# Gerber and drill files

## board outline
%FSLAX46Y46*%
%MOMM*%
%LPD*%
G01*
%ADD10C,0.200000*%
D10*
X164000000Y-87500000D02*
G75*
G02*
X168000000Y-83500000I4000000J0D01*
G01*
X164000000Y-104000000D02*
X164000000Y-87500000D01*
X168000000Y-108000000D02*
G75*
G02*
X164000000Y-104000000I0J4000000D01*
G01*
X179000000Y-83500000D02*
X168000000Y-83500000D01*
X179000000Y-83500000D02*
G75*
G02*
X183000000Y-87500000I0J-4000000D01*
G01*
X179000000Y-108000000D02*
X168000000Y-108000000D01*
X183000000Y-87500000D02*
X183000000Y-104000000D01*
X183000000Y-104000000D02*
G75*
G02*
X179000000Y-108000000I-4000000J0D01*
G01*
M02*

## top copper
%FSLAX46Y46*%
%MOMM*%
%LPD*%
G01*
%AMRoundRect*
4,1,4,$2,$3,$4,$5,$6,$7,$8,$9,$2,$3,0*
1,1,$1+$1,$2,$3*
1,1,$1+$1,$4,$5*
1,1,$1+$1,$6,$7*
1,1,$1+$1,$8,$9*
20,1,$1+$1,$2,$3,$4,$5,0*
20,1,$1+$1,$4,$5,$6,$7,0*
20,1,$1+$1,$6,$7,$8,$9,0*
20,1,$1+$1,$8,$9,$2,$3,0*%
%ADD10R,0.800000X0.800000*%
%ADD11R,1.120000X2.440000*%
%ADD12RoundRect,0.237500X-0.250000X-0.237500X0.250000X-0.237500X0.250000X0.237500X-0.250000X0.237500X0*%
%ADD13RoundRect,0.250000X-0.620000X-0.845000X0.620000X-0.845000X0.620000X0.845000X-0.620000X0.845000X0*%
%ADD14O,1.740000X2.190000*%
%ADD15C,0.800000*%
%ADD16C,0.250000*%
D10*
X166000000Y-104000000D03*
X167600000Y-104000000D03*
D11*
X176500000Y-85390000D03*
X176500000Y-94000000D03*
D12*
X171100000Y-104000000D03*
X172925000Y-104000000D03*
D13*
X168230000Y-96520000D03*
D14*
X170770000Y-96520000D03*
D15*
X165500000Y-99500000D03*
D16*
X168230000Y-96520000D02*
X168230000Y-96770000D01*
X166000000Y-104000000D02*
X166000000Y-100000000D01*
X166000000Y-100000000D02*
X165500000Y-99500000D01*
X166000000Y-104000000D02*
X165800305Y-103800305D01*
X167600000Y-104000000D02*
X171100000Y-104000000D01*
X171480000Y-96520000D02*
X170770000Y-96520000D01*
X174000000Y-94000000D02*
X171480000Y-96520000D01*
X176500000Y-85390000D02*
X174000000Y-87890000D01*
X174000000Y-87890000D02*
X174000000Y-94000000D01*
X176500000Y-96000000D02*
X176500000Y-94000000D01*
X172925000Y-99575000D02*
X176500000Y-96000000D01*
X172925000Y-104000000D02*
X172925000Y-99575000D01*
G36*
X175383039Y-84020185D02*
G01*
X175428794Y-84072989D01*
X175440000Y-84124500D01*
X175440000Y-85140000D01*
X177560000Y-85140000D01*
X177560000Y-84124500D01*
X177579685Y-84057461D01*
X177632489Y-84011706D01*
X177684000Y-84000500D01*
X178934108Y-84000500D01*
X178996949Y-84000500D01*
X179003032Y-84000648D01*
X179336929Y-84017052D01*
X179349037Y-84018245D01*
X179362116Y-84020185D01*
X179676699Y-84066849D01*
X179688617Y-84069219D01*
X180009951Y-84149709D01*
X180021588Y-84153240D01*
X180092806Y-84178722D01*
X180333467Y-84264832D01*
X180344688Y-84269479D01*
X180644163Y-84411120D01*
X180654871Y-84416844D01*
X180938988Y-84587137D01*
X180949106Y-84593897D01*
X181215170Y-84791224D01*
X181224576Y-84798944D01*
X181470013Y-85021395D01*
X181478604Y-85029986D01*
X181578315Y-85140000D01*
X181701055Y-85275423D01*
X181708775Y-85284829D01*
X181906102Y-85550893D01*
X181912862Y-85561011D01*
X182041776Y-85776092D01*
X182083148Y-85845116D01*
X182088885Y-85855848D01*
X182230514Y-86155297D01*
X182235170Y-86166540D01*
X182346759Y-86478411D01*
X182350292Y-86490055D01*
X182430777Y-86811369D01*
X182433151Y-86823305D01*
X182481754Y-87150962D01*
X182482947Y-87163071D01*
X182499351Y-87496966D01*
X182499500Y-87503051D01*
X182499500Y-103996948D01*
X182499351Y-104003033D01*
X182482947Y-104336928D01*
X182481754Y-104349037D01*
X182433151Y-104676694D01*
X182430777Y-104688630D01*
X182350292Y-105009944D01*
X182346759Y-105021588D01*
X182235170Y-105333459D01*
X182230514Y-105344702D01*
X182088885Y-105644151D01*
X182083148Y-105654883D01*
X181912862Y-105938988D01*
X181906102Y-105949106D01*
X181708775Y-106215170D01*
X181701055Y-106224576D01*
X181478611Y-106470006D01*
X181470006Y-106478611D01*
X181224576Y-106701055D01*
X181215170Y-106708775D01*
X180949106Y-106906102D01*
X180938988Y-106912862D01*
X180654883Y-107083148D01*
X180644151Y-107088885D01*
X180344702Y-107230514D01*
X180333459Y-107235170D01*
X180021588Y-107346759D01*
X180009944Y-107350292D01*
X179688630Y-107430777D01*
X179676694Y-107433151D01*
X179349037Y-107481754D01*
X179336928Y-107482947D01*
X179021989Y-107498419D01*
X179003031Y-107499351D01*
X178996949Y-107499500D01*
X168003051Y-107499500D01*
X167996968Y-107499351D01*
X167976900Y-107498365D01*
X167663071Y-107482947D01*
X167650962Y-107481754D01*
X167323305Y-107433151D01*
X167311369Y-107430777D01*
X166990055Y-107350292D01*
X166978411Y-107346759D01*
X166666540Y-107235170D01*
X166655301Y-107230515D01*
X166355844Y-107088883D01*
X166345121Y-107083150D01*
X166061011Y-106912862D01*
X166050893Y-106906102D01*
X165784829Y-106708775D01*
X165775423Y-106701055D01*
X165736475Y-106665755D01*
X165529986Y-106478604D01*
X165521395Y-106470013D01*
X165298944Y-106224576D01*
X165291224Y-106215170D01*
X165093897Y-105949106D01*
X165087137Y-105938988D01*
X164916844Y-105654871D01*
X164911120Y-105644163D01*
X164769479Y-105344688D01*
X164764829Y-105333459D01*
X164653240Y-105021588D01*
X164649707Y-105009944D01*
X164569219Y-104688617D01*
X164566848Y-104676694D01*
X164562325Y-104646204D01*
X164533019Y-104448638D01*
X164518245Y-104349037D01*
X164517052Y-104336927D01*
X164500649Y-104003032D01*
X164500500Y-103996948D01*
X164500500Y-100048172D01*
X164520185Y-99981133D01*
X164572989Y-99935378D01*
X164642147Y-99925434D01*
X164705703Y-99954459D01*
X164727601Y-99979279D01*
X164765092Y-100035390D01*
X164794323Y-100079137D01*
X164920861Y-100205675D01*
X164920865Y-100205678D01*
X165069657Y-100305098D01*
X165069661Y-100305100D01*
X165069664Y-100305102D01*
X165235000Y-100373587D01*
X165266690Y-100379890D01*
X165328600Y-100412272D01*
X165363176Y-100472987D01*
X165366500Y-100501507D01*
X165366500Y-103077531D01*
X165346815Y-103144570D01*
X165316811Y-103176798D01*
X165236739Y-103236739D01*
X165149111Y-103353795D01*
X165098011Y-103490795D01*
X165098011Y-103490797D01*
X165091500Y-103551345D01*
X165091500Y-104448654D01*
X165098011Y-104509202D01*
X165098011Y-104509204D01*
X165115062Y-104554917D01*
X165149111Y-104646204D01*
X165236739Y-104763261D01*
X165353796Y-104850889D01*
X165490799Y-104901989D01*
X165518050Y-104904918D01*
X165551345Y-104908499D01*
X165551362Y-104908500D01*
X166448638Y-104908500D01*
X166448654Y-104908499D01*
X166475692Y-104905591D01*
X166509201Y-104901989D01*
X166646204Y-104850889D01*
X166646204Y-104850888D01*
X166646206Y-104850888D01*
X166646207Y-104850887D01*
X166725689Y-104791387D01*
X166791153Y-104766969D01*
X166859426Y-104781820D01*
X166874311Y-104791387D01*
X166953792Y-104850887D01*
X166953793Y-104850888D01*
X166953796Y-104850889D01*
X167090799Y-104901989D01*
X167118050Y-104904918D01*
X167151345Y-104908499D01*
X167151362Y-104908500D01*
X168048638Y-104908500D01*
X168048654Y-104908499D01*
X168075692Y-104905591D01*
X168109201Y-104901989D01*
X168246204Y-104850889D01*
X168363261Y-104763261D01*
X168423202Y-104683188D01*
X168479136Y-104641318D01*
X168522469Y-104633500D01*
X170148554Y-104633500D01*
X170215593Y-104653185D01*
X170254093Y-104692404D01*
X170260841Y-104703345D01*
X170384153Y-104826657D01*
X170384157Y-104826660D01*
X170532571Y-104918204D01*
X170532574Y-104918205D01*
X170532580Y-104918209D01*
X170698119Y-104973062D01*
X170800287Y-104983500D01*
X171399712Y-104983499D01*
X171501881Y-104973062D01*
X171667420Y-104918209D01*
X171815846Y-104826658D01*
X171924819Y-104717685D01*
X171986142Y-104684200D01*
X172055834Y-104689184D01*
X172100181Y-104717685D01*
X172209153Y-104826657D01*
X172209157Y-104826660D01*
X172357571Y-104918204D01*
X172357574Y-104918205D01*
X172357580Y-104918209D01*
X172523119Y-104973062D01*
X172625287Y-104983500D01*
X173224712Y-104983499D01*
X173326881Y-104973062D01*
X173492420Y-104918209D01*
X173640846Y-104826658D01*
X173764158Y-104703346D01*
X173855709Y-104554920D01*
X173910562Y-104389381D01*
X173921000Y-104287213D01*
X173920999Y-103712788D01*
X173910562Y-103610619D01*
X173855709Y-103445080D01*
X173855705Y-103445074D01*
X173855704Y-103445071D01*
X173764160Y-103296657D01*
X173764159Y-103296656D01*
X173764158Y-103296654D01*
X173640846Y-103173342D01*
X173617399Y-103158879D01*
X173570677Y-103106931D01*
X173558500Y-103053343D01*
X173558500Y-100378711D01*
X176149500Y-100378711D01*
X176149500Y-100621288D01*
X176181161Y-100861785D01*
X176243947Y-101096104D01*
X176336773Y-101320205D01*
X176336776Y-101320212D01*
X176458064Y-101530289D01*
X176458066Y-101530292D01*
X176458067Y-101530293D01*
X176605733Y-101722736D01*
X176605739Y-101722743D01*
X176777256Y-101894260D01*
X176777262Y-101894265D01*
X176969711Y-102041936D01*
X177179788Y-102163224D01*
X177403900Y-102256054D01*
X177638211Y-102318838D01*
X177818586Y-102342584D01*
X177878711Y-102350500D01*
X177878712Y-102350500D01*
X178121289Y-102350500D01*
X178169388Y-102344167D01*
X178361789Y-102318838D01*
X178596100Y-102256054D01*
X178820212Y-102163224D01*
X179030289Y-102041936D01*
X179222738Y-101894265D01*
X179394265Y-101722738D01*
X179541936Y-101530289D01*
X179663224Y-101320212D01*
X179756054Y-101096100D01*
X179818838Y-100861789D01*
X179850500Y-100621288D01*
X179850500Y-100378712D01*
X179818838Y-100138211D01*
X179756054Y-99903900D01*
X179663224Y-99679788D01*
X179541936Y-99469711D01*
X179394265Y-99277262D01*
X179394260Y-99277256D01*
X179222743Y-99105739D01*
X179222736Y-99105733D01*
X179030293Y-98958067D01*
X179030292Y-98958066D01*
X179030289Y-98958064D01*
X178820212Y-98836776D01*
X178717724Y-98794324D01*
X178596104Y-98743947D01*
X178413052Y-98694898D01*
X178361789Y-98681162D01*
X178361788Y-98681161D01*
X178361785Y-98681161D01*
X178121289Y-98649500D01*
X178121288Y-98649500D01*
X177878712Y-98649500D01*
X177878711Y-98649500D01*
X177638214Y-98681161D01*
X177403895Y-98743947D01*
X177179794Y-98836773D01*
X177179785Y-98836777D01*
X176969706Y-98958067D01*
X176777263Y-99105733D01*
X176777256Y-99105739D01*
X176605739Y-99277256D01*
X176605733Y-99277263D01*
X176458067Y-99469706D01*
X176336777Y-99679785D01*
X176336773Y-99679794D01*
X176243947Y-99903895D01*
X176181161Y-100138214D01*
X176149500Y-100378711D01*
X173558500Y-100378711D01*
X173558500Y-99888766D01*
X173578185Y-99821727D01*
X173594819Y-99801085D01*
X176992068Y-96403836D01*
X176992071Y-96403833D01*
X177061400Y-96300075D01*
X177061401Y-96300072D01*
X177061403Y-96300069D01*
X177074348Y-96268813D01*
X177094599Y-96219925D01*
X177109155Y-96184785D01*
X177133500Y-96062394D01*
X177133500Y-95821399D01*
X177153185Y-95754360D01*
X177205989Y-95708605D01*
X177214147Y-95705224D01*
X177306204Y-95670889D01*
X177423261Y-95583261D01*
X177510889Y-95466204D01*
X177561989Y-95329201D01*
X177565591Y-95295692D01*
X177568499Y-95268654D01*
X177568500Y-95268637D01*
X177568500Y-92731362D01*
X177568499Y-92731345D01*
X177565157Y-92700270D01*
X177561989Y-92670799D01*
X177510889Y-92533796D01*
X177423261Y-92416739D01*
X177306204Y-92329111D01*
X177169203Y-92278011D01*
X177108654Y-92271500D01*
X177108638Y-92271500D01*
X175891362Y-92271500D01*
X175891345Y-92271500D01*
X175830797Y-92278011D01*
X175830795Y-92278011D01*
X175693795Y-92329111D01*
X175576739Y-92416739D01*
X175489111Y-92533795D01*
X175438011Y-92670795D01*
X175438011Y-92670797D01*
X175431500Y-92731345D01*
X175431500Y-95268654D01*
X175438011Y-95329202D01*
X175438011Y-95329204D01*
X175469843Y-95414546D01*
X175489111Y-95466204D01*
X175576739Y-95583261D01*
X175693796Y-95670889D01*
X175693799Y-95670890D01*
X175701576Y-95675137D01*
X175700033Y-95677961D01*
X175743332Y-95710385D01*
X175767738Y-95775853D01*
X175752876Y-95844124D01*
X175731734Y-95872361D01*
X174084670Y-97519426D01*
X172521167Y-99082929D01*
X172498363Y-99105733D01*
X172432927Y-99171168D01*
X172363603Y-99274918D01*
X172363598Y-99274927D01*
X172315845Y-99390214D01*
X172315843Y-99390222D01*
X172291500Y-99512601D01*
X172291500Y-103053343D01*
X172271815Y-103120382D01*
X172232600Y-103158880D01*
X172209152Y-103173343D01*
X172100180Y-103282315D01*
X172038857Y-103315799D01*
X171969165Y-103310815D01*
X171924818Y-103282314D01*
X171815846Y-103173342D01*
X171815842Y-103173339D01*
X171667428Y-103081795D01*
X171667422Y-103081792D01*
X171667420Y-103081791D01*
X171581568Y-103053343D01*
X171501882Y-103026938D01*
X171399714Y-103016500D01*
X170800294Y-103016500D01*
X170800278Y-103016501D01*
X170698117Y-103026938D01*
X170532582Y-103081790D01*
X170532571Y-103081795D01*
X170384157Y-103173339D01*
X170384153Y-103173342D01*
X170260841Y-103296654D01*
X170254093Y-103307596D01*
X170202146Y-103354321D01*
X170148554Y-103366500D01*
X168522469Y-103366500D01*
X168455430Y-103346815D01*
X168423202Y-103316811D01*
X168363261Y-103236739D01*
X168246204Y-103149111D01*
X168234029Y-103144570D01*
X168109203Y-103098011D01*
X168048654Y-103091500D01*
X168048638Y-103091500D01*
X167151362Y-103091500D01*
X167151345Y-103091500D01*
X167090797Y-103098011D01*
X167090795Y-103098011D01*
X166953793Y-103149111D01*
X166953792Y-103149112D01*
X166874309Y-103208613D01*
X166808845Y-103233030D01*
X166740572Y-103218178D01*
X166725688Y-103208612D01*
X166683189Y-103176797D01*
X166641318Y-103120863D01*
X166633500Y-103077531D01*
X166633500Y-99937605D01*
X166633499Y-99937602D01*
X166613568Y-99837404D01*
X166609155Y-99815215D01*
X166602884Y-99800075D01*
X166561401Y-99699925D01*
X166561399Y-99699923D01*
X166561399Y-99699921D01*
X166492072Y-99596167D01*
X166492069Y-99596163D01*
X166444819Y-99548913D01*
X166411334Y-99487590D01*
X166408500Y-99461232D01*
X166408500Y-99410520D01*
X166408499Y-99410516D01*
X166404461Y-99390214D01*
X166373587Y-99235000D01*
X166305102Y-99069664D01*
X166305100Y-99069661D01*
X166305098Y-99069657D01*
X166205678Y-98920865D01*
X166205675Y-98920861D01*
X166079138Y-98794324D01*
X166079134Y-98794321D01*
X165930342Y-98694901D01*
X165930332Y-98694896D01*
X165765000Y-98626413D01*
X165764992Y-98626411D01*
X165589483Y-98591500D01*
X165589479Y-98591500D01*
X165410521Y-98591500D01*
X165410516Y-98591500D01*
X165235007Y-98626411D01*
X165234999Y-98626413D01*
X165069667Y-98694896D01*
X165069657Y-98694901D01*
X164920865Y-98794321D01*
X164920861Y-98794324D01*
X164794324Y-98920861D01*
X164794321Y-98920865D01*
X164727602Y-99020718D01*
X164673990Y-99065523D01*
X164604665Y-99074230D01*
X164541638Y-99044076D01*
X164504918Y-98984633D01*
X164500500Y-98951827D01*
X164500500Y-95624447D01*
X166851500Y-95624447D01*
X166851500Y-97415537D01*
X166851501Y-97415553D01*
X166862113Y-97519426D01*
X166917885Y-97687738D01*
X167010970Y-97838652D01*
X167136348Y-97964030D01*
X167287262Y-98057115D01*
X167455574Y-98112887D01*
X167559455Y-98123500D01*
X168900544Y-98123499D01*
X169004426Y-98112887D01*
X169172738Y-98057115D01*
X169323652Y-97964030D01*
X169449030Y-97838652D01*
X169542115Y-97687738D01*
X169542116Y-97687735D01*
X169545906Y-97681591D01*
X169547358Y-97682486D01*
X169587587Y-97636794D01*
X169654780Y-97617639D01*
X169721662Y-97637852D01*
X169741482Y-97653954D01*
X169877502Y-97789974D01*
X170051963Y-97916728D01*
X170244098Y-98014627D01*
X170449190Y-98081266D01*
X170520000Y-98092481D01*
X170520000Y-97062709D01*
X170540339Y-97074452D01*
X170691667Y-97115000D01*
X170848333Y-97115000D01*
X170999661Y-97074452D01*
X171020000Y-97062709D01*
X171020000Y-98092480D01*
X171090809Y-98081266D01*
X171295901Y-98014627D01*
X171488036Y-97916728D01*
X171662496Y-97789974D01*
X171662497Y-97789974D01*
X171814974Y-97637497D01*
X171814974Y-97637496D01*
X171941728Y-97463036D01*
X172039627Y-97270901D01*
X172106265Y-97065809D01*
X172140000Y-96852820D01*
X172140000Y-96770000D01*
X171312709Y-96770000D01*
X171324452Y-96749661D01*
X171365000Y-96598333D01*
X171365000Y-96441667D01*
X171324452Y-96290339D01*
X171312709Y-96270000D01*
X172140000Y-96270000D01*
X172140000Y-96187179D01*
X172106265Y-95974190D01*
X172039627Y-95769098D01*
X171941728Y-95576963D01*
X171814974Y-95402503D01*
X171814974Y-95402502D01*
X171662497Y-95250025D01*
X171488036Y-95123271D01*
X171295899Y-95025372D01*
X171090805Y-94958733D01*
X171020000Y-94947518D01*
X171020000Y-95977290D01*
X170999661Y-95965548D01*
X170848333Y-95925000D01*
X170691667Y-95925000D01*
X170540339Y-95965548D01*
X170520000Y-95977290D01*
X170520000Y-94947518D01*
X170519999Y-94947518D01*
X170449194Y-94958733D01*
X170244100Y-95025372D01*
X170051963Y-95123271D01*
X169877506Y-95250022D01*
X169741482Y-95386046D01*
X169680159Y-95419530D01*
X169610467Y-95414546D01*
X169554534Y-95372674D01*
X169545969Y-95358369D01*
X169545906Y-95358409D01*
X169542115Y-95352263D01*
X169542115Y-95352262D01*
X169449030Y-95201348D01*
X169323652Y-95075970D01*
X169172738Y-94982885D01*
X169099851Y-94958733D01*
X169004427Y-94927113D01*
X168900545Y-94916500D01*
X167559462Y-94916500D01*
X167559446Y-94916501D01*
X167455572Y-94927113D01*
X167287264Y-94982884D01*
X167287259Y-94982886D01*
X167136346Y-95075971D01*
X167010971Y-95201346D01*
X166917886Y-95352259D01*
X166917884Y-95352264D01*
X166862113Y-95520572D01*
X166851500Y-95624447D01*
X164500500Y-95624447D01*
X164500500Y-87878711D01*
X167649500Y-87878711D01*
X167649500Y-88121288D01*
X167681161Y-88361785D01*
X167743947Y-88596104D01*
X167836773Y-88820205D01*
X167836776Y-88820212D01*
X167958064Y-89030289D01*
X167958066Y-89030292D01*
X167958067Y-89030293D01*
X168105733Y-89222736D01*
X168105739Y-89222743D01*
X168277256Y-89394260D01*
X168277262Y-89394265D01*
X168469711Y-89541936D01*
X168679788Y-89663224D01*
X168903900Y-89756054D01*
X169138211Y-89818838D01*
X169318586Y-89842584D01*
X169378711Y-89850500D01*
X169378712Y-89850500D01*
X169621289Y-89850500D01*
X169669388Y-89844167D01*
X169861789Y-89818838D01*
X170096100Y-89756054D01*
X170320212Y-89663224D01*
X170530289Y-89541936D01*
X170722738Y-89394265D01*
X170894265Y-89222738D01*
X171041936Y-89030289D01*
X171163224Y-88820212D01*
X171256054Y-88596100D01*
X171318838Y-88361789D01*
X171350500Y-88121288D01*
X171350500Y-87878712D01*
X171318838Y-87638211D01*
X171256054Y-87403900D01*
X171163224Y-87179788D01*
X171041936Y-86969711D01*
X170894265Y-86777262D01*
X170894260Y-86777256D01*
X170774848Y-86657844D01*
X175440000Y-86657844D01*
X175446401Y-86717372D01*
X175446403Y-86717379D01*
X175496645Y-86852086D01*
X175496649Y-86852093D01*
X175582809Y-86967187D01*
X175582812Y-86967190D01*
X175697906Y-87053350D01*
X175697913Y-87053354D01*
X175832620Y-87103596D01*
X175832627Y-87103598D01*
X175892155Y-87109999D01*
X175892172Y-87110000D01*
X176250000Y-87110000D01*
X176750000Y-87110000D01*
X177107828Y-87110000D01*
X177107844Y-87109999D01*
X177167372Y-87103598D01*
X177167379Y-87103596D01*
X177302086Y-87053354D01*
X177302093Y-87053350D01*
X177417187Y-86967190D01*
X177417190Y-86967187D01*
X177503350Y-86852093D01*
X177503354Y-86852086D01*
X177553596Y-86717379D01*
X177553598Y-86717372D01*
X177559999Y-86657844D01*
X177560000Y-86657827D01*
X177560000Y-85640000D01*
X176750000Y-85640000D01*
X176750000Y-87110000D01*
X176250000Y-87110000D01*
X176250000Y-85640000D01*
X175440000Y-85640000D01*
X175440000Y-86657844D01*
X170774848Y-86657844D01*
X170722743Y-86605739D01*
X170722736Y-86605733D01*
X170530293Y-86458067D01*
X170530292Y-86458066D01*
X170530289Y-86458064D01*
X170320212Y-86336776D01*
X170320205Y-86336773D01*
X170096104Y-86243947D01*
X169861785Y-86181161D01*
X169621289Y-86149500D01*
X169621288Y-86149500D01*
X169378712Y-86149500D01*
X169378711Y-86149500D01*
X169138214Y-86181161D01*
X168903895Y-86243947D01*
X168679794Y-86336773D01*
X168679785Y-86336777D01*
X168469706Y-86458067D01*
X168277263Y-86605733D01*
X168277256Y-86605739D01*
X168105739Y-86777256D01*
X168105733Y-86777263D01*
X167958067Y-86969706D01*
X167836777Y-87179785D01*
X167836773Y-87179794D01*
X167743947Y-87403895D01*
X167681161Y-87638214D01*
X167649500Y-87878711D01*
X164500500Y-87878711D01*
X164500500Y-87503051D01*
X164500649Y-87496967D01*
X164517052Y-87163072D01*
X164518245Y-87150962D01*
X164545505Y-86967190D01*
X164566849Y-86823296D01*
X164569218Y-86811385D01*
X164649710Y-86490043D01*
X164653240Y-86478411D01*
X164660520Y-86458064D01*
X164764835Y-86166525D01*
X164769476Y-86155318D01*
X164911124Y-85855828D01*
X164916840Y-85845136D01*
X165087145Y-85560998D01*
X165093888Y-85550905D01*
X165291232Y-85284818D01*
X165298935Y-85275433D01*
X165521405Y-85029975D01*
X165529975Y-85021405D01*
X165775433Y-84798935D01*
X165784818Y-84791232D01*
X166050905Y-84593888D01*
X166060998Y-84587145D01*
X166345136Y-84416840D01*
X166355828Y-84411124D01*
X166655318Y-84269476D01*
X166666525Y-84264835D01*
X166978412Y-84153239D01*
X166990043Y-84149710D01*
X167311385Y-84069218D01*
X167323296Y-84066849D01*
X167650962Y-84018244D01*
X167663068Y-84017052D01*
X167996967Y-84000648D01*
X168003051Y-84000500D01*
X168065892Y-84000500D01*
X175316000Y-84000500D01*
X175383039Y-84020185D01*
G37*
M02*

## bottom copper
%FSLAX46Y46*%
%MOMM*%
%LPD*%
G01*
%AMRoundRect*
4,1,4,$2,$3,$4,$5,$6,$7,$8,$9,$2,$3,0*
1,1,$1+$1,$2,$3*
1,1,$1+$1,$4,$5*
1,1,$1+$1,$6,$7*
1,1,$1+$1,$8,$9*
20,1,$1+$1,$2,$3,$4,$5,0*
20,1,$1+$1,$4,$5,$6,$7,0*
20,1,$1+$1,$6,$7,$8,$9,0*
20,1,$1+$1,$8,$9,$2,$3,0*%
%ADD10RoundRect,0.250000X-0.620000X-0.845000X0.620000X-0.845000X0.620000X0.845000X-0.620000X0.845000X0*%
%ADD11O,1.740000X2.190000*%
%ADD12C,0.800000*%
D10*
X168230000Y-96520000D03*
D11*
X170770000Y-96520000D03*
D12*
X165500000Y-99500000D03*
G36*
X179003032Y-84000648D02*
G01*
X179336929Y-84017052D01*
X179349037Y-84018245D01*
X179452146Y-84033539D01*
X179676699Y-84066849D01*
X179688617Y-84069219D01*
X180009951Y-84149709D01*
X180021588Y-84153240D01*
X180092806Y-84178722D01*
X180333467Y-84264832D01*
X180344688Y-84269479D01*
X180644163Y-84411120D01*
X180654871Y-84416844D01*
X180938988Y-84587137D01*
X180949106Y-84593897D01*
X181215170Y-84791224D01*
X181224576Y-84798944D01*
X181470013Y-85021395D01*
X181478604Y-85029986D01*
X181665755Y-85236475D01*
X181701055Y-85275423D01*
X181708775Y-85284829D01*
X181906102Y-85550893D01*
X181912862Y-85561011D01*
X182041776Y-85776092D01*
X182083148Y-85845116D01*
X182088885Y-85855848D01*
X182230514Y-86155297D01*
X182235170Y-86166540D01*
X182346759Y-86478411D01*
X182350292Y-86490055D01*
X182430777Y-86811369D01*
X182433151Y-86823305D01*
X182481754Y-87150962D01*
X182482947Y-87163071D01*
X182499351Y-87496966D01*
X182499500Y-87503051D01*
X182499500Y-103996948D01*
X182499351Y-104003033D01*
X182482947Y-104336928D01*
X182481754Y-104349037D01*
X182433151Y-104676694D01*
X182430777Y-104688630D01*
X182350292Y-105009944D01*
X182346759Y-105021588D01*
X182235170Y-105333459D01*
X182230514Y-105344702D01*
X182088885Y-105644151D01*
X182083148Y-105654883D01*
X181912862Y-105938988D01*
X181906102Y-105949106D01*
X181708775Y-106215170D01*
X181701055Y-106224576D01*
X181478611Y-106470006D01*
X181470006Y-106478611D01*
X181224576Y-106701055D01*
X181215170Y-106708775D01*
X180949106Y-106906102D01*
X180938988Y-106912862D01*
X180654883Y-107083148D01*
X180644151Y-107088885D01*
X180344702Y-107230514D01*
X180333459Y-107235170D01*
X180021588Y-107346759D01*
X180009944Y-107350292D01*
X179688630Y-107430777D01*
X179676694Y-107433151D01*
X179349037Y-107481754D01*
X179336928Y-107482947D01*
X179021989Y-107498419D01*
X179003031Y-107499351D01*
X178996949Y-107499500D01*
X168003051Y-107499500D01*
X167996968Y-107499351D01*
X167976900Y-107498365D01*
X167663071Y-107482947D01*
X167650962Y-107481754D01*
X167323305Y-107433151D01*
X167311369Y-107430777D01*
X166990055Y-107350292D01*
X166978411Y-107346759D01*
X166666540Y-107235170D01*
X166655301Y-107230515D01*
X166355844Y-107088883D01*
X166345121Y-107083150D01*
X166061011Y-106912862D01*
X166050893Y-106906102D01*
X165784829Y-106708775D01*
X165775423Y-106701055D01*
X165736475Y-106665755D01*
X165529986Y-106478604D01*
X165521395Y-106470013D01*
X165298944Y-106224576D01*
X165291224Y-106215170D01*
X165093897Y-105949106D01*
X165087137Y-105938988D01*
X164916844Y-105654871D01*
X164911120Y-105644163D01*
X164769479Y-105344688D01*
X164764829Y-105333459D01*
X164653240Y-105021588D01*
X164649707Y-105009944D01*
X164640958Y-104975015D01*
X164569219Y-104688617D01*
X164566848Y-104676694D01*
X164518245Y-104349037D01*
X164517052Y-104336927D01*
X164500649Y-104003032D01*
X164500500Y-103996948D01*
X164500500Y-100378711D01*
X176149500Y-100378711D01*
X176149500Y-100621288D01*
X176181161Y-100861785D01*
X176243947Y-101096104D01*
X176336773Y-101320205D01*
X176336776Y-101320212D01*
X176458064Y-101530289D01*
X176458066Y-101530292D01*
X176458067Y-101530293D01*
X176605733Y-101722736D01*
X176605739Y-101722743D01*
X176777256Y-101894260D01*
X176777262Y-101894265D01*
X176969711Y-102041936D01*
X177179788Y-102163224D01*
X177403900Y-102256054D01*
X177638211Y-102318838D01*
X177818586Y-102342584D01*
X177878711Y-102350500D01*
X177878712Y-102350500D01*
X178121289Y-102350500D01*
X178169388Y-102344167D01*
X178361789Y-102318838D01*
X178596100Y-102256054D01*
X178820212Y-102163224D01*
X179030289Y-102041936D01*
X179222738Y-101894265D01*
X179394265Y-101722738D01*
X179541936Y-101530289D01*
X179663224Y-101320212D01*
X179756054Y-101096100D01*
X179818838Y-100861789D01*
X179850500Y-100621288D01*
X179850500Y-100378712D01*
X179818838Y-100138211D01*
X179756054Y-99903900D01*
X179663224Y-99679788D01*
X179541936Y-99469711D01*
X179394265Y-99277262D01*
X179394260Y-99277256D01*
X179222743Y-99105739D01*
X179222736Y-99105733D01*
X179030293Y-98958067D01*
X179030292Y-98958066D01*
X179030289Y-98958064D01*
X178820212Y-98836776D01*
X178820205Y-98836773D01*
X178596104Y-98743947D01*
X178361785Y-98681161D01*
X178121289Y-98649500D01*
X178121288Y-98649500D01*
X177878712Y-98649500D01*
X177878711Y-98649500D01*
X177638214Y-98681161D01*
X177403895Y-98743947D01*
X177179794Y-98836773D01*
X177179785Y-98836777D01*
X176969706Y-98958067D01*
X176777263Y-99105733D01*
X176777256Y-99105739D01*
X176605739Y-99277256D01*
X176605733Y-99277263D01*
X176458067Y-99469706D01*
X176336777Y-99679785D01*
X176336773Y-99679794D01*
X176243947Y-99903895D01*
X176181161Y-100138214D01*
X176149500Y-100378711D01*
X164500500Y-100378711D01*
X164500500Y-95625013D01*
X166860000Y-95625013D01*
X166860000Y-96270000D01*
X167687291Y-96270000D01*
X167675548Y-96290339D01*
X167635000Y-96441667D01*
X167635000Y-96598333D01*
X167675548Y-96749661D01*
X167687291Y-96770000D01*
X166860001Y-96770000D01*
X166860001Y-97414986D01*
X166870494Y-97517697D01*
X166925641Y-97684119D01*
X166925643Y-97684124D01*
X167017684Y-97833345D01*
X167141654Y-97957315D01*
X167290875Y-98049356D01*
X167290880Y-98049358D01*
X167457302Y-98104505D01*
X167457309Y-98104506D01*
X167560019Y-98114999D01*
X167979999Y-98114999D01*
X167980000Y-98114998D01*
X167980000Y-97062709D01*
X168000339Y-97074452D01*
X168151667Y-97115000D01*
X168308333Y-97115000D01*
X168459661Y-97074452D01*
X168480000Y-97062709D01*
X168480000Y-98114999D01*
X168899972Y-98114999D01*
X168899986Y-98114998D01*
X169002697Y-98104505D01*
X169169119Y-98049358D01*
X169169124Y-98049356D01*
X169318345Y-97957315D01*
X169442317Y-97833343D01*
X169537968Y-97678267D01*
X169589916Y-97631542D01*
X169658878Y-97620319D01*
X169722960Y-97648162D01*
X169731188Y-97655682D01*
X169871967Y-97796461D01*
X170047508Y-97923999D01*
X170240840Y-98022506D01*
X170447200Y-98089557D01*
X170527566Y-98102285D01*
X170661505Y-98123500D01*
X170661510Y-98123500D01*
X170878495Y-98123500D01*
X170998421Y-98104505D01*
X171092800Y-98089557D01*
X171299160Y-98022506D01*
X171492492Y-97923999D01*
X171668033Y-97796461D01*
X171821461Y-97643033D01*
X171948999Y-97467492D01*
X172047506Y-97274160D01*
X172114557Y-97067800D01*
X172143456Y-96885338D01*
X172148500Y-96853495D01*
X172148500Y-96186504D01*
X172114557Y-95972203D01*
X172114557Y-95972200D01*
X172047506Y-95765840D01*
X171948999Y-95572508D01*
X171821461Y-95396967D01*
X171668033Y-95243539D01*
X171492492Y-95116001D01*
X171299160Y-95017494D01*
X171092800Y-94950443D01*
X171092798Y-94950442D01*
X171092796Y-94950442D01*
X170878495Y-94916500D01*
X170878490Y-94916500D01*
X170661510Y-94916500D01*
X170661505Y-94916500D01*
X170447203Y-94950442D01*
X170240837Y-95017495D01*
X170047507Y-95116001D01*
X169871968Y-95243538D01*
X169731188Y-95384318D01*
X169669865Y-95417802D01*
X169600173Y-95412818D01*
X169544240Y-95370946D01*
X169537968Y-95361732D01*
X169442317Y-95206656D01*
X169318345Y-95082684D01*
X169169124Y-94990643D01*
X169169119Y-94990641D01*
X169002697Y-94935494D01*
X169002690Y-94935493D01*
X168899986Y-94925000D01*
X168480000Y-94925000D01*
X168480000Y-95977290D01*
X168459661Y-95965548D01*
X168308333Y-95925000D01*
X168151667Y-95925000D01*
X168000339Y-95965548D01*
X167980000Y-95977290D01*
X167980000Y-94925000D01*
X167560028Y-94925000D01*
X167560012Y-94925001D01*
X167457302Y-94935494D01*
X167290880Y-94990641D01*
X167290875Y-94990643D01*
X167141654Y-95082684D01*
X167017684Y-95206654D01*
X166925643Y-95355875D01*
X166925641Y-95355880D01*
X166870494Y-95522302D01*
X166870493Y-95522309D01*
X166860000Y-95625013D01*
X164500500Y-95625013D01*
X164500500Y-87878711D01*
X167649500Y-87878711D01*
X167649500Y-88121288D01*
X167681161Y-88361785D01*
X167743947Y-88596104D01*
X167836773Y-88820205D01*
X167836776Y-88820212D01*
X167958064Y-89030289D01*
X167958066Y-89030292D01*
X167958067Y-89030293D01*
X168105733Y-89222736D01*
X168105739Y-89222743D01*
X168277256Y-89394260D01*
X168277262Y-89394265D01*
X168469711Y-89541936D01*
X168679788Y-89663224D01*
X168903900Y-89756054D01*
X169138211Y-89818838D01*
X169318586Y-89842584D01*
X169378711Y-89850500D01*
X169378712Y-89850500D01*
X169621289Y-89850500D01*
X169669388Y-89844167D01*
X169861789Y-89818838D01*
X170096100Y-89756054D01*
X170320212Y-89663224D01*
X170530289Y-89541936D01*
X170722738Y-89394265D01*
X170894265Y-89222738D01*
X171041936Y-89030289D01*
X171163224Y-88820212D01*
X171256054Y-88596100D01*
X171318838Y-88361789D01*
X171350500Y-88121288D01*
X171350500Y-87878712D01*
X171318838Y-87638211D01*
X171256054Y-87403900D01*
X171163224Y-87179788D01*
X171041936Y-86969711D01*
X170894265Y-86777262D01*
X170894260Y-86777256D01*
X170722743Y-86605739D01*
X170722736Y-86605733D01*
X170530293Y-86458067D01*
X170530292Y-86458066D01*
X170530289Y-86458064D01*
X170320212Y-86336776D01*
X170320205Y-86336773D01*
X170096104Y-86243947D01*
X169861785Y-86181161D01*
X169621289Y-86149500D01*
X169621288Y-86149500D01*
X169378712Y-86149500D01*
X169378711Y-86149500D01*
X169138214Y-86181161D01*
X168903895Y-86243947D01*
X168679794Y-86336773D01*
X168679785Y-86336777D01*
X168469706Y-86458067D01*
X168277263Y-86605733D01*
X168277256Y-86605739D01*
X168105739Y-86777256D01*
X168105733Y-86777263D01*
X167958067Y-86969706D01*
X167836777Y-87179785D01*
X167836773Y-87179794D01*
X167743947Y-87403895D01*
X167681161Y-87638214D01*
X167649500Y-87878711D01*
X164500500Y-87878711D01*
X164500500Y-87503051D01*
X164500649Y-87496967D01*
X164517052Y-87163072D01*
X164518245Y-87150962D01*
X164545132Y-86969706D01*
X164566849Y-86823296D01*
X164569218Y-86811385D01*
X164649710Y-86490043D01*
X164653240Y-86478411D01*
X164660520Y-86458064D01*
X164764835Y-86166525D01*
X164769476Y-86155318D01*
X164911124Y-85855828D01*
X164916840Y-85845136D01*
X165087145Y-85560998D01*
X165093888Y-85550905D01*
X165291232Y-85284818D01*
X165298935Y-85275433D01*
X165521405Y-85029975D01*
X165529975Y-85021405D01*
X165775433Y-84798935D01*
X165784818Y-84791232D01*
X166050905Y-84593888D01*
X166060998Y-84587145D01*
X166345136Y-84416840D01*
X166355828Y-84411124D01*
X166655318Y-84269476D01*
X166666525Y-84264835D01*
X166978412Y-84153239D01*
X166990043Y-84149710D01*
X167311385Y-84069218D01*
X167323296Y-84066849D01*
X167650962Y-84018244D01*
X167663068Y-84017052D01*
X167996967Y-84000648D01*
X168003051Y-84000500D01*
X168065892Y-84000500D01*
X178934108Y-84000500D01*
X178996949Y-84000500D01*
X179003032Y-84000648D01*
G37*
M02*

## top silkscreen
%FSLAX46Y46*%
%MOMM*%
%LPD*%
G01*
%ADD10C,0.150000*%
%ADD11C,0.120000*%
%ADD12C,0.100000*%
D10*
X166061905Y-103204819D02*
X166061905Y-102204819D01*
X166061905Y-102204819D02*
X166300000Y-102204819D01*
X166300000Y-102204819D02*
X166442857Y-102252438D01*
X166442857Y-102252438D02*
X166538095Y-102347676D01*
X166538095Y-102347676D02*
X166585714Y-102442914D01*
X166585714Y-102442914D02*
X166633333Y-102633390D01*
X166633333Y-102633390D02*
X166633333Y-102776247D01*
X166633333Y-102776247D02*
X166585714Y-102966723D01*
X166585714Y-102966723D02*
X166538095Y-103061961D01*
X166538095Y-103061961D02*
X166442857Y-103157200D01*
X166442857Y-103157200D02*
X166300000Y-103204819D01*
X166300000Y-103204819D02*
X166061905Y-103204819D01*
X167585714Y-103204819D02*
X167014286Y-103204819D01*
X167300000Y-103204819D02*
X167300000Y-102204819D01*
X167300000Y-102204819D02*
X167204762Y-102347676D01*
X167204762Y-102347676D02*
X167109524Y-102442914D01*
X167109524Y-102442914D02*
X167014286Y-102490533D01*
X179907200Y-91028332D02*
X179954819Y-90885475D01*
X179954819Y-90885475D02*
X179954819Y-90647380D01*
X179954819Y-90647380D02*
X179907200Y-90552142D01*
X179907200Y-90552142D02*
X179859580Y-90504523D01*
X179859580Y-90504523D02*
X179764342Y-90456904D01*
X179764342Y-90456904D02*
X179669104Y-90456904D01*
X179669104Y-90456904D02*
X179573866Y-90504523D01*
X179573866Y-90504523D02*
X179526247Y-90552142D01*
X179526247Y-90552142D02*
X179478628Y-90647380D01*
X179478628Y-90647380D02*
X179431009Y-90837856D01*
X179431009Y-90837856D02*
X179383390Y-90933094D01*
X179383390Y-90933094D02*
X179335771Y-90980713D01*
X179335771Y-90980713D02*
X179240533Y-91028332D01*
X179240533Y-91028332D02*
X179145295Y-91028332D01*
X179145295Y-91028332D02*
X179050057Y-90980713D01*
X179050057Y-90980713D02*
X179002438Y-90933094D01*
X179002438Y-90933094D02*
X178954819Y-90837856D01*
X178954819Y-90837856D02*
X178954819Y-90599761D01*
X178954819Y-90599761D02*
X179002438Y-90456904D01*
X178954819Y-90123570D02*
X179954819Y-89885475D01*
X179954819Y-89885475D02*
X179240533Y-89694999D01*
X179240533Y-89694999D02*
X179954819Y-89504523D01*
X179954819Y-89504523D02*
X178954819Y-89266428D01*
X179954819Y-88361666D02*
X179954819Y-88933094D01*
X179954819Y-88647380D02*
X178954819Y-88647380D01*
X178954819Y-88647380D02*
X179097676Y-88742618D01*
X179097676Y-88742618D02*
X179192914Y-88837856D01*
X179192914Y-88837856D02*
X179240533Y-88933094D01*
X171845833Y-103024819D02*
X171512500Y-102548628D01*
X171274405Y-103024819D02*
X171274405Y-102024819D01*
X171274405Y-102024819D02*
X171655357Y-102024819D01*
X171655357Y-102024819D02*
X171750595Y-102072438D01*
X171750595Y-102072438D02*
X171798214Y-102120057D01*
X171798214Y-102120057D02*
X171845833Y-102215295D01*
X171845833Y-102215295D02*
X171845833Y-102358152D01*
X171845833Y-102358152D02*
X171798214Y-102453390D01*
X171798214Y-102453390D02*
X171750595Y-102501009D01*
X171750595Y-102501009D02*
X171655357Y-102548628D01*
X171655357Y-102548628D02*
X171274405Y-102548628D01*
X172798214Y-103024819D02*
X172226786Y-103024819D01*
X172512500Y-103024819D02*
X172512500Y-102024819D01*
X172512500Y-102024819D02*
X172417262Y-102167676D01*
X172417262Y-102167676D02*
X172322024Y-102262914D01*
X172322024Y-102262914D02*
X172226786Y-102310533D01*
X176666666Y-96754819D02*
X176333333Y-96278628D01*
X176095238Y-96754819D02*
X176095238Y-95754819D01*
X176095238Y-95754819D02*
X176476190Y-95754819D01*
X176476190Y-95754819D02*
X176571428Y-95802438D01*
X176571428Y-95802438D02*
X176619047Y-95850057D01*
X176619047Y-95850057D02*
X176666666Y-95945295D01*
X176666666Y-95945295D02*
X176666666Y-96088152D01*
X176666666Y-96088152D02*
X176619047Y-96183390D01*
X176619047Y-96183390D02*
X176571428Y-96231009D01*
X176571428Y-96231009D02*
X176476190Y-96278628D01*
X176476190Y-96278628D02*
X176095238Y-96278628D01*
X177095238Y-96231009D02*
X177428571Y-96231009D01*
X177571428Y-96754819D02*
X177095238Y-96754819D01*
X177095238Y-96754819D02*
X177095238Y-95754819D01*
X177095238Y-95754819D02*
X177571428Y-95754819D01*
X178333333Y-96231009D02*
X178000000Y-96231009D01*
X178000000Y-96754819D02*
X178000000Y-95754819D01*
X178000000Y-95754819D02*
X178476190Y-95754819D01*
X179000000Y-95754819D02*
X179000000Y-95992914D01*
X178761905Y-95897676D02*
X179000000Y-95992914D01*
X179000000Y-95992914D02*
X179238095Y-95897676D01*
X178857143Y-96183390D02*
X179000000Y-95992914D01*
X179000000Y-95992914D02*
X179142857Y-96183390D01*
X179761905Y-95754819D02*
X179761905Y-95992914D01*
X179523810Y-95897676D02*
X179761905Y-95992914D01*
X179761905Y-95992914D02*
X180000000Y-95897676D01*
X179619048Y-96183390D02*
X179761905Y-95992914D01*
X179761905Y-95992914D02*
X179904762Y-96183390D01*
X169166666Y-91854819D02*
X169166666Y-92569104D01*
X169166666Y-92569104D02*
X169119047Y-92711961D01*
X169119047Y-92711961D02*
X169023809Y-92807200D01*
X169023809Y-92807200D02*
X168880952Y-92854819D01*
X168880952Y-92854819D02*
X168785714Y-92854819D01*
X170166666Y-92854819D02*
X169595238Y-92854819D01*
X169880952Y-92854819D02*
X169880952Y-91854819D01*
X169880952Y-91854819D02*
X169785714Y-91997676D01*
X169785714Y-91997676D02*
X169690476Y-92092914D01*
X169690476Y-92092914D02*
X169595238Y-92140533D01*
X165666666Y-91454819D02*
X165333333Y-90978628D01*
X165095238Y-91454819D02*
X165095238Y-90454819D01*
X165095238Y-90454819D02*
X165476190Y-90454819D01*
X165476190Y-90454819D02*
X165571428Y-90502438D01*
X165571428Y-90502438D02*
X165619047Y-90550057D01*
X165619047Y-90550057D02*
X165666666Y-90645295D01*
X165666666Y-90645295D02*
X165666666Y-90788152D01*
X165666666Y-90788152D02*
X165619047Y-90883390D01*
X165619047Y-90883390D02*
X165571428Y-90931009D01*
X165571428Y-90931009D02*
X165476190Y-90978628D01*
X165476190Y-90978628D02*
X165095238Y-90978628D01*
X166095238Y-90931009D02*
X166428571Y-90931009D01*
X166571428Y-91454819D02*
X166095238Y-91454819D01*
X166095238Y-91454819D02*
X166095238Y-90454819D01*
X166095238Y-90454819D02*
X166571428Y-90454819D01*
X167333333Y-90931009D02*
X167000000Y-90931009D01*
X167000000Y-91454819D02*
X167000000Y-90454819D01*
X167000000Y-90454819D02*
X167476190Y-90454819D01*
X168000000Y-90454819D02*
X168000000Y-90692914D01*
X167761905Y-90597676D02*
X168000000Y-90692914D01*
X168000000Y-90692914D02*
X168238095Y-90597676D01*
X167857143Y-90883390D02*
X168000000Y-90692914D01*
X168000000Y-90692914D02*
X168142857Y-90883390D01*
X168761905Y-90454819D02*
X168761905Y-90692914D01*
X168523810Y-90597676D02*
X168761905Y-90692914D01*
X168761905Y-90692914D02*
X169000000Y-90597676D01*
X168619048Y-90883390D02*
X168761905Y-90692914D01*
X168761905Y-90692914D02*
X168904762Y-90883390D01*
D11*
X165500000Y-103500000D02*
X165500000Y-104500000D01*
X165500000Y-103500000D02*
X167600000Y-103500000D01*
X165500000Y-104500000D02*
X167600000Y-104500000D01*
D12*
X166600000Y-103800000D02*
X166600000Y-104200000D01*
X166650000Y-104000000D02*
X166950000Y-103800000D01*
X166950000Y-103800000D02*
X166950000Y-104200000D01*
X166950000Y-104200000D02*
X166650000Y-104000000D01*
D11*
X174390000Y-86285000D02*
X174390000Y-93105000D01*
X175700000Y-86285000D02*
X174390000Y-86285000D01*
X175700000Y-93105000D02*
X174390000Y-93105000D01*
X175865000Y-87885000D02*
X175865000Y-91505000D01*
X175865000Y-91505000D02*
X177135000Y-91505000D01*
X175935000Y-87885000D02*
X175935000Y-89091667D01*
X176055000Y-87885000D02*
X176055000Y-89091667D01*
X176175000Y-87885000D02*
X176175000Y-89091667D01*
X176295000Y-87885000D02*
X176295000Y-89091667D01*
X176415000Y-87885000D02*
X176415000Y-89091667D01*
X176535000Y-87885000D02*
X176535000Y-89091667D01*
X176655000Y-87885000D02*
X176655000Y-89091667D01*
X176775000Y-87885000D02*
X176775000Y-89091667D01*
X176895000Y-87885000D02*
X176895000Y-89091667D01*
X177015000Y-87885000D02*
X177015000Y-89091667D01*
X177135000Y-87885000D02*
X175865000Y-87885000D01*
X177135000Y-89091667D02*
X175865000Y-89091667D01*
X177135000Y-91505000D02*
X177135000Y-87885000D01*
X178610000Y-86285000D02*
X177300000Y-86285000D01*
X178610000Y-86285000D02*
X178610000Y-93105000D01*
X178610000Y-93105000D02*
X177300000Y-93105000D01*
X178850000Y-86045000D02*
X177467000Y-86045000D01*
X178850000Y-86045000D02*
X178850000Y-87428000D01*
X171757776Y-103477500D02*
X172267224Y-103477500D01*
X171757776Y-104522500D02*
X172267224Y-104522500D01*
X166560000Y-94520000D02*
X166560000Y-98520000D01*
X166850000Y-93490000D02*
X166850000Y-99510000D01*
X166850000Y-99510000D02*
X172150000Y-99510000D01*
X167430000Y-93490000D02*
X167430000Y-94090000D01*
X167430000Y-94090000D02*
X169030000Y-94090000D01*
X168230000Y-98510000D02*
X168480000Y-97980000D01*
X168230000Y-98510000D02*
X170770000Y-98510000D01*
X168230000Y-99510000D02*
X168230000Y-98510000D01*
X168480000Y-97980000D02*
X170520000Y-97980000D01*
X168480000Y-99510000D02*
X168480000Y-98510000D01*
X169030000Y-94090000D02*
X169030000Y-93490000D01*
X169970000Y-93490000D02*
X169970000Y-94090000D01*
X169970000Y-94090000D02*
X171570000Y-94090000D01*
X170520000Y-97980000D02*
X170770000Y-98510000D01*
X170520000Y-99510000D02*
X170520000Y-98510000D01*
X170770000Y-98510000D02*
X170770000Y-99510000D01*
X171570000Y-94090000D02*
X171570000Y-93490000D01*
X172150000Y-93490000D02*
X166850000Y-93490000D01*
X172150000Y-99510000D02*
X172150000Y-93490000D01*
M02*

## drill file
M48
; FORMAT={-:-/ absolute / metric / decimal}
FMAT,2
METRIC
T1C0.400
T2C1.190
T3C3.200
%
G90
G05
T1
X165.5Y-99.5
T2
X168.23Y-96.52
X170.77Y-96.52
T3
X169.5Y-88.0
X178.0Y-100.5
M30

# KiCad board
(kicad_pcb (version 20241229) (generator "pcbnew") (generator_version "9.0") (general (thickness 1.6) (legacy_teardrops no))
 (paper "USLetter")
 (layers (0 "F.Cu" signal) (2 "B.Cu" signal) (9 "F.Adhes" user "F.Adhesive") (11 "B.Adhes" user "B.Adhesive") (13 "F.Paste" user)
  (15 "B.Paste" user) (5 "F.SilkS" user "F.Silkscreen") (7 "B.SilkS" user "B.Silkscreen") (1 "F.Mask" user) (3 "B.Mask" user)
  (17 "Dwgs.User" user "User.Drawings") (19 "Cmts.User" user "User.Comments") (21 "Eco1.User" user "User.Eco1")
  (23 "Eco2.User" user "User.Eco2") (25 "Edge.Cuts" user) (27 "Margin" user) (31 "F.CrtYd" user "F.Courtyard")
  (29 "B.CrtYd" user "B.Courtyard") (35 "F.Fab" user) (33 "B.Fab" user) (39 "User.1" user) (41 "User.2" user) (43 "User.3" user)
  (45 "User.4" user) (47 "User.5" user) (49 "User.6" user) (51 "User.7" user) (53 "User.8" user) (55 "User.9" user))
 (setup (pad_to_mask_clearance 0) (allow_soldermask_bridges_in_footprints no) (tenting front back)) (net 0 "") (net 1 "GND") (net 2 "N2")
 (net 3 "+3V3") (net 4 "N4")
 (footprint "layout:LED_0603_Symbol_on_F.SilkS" (layer "F.Cu") (at 166.8 104)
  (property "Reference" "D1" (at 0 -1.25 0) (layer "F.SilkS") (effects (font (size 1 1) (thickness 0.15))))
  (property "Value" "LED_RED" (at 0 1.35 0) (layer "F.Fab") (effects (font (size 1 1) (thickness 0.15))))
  (fp_line (start -1.3 -0.5) (end -1.3 0.5) (stroke (width 0.12) (type solid)) (layer "F.SilkS"))
  (fp_line (start -1.3 -0.5) (end 0.8 -0.5) (stroke (width 0.12) (type solid)) (layer "F.SilkS"))
  (fp_line (start -1.3 0.5) (end 0.8 0.5) (stroke (width 0.12) (type solid)) (layer "F.SilkS"))
  (fp_line (start -0.2 -0.2) (end -0.2 0.2) (stroke (width 0.1) (type solid)) (layer "F.SilkS"))
  (fp_line (start -0.15 0) (end 0.15 -0.2) (stroke (width 0.1) (type solid)) (layer "F.SilkS"))
  (fp_line (start 0.15 -0.2) (end 0.15 0.2) (stroke (width 0.1) (type solid)) (layer "F.SilkS"))
  (fp_line (start 0.15 0.2) (end -0.15 0) (stroke (width 0.1) (type solid)) (layer "F.SilkS"))
  (pad "1" smd rect (at -0.8 0 180) (size 0.8 0.8) (layers "F.Cu" "F.Mask" "F.Paste") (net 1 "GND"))
  (pad "2" smd rect (at 0.8 0 180) (size 0.8 0.8) (layers "F.Cu" "F.Mask" "F.Paste") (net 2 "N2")))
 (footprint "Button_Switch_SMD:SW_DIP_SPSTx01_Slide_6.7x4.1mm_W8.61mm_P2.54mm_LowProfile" (layer "F.Cu") (at 176.5 89.695 -90)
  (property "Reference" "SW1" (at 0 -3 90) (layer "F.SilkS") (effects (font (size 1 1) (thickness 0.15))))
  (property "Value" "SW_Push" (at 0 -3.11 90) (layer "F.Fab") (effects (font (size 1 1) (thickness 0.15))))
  (fp_line (start -3.41 2.11) (end 3.41 2.11) (stroke (width 0.12) (type solid)) (layer "F.SilkS"))
  (fp_line (start -3.41 0.8) (end -3.41 2.11) (stroke (width 0.12) (type solid)) (layer "F.SilkS"))
  (fp_line (start 3.41 0.8) (end 3.41 2.11) (stroke (width 0.12) (type solid)) (layer "F.SilkS"))
  (fp_line (start -1.81 0.635) (end 1.81 0.635) (stroke (width 0.12) (type solid)) (layer "F.SilkS"))
  (fp_line (start 1.81 0.635) (end 1.81 -0.635) (stroke (width 0.12) (type solid)) (layer "F.SilkS"))
  (fp_line (start -1.81 0.565) (end -0.603333 0.565) (stroke (width 0.12) (type solid)) (layer "F.SilkS"))
  (fp_line (start -1.81 0.445) (end -0.603333 0.445) (stroke (width 0.12) (type solid)) (layer "F.SilkS"))
  (fp_line (start -1.81 0.325) (end -0.603333 0.325) (stroke (width 0.12) (type solid)) (layer "F.SilkS"))
  (fp_line (start -1.81 0.205) (end -0.603333 0.205) (stroke (width 0.12) (type solid)) (layer "F.SilkS"))
  (fp_line (start -1.81 0.085) (end -0.603333 0.085) (stroke (width 0.12) (type solid)) (layer "F.SilkS"))
  (fp_line (start -1.81 -0.035) (end -0.603333 -0.035) (stroke (width 0.12) (type solid)) (layer "F.SilkS"))
  (fp_line (start -1.81 -0.155) (end -0.603333 -0.155) (stroke (width 0.12) (type solid)) (layer "F.SilkS"))
  (fp_line (start -1.81 -0.275) (end -0.603333 -0.275) (stroke (width 0.12) (type solid)) (layer "F.SilkS"))
  (fp_line (start -1.81 -0.395) (end -0.603333 -0.395) (stroke (width 0.12) (type solid)) (layer "F.SilkS"))
  (fp_line (start -1.81 -0.515) (end -0.603333 -0.515) (stroke (width 0.12) (type solid)) (layer "F.SilkS"))
  (fp_line (start -1.81 -0.635) (end -1.81 0.635) (stroke (width 0.12) (type solid)) (layer "F.SilkS"))
  (fp_line (start -0.603333 -0.635) (end -0.603333 0.635) (stroke (width 0.12) (type solid)) (layer "F.SilkS"))
  (fp_line (start 1.81 -0.635) (end -1.81 -0.635) (stroke (width 0.12) (type solid)) (layer "F.SilkS"))
  (fp_line (start -3.41 -2.11) (end -3.41 -0.8) (stroke (width 0.12) (type solid)) (layer "F.SilkS"))
  (fp_line (start -3.41 -2.11) (end 3.41 -2.11) (stroke (width 0.12) (type solid)) (layer "F.SilkS"))
  (fp_line (start 3.41 -2.11) (end 3.41 -0.8) (stroke (width 0.12) (type solid)) (layer "F.SilkS"))
  (fp_line (start -3.65 -2.35) (end -3.65 -0.967) (stroke (width 0.12) (type solid)) (layer "F.SilkS"))
  (fp_line (start -3.65 -2.35) (end -2.267 -2.35) (stroke (width 0.12) (type solid)) (layer "F.SilkS"))
  (pad "1" smd rect (at -4.305 0 270) (size 2.44 1.12) (layers "F.Cu" "F.Mask" "F.Paste") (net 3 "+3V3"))
  (pad "2" smd rect (at 4.305 0 270) (size 2.44 1.12) (layers "F.Cu" "F.Mask" "F.Paste") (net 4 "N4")))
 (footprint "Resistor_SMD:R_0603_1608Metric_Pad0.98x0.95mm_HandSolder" (layer "F.Cu") (at 172.0125 104)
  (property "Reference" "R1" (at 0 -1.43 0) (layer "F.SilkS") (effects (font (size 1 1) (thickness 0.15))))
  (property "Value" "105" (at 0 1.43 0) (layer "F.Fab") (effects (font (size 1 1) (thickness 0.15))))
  (fp_line (start -0.254724 -0.5225) (end 0.254724 -0.5225) (stroke (width 0.12) (type solid)) (layer "F.SilkS"))
  (fp_line (start -0.254724 0.5225) (end 0.254724 0.5225) (stroke (width 0.12) (type solid)) (layer "F.SilkS"))
  (pad "1" smd roundrect (at -0.9125 0) (size 0.975 0.95) (layers "F.Cu" "F.Mask" "F.Paste") (roundrect_rratio 0.25) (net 2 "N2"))
  (pad "2" smd roundrect (at 0.9125 0) (size 0.975 0.95) (layers "F.Cu" "F.Mask" "F.Paste") (roundrect_rratio 0.25) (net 4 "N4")))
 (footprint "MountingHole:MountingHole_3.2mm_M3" (layer "F.Cu") (at 178 100.5)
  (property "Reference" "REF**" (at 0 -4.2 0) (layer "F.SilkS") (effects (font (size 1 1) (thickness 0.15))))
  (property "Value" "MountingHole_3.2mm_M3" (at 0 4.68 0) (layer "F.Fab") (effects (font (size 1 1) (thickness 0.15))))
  (pad "" np_thru_hole circle (at 0 0) (size 3.2 3.2) (drill 3.2) (layers "*.Cu" "*.Mask")))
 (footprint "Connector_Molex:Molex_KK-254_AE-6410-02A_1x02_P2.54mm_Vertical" (layer "F.Cu") (at 168.23 96.52)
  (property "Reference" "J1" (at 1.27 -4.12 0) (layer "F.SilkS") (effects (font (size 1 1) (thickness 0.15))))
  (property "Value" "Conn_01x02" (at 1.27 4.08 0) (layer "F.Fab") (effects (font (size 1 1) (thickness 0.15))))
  (fp_line (start -1.67 -2) (end -1.67 2) (stroke (width 0.12) (type solid)) (layer "F.SilkS"))
  (fp_line (start -1.38 -3.03) (end -1.38 2.99) (stroke (width 0.12) (type solid)) (layer "F.SilkS"))
  (fp_line (start -1.38 2.99) (end 3.92 2.99) (stroke (width 0.12) (type solid)) (layer "F.SilkS"))
  (fp_line (start -0.8 -3.03) (end -0.8 -2.43) (stroke (width 0.12) (type solid)) (layer "F.SilkS"))
  (fp_line (start -0.8 -2.43) (end 0.8 -2.43) (stroke (width 0.12) (type solid)) (layer "F.SilkS"))
  (fp_line (start 0 1.99) (end 0.25 1.46) (stroke (width 0.12) (type solid)) (layer "F.SilkS"))
  (fp_line (start 0 1.99) (end 2.54 1.99) (stroke (width 0.12) (type solid)) (layer "F.SilkS"))
  (fp_line (start 0 2.99) (end 0 1.99) (stroke (width 0.12) (type solid)) (layer "F.SilkS"))
  (fp_line (start 0.25 1.46) (end 2.29 1.46) (stroke (width 0.12) (type solid)) (layer "F.SilkS"))
  (fp_line (start 0.25 2.99) (end 0.25 1.99) (stroke (width 0.12) (type solid)) (layer "F.SilkS"))
  (fp_line (start 0.8 -2.43) (end 0.8 -3.03) (stroke (width 0.12) (type solid)) (layer "F.SilkS"))
  (fp_line (start 1.74 -3.03) (end 1.74 -2.43) (stroke (width 0.12) (type solid)) (layer "F.SilkS"))
  (fp_line (start 1.74 -2.43) (end 3.34 -2.43) (stroke (width 0.12) (type solid)) (layer "F.SilkS"))
  (fp_line (start 2.29 1.46) (end 2.54 1.99) (stroke (width 0.12) (type solid)) (layer "F.SilkS"))
  (fp_line (start 2.29 2.99) (end 2.29 1.99) (stroke (width 0.12) (type solid)) (layer "F.SilkS"))
  (fp_line (start 2.54 1.99) (end 2.54 2.99) (stroke (width 0.12) (type solid)) (layer "F.SilkS"))
  (fp_line (start 3.34 -2.43) (end 3.34 -3.03) (stroke (width 0.12) (type solid)) (layer "F.SilkS"))
  (fp_line (start 3.92 -3.03) (end -1.38 -3.03) (stroke (width 0.12) (type solid)) (layer "F.SilkS"))
  (fp_line (start 3.92 2.99) (end 3.92 -3.03) (stroke (width 0.12) (type solid)) (layer "F.SilkS"))
  (pad "1" thru_hole roundrect (at 0 0) (size 1.74 2.19) (drill 1.19) (layers "*.Cu" "*.Mask") (remove_unused_layers no)
   (roundrect_rratio 0.143678) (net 1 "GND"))
  (pad "2" thru_hole oval (at 2.54 0) (size 1.74 2.19) (drill 1.19) (layers "*.Cu" "*.Mask") (remove_unused_layers no) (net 3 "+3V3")))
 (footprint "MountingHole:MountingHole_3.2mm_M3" (layer "F.Cu") (at 169.5 88)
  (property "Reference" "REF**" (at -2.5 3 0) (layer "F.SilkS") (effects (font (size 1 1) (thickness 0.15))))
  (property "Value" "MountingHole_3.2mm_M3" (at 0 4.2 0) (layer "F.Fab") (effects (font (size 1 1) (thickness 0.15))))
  (pad "" np_thru_hole circle (at 0 0) (size 3.2 3.2) (drill 3.2) (layers "*.Cu" "*.Mask")))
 (gr_arc (start 164 87.5) (mid 165.171573 84.671573) (end 168 83.5) (stroke (width 0.2) (type solid)) (layer "Edge.Cuts"))
 (gr_line (start 164 104) (end 164 87.5) (stroke (width 0.2) (type solid)) (layer "Edge.Cuts"))
 (gr_arc (start 168 108) (mid 165.171573 106.828427) (end 164 104) (stroke (width 0.2) (type solid)) (layer "Edge.Cuts"))
 (gr_line (start 179 83.5) (end 168 83.5) (stroke (width 0.2) (type solid)) (layer "Edge.Cuts"))
 (gr_arc (start 179 83.5) (mid 181.828427 84.671573) (end 183 87.5) (stroke (width 0.2) (type solid)) (layer "Edge.Cuts"))
 (gr_line (start 179 108) (end 168 108) (stroke (width 0.2) (type solid)) (layer "Edge.Cuts"))
 (gr_line (start 183 87.5) (end 183 104) (stroke (width 0.2) (type solid)) (layer "Edge.Cuts"))
 (gr_arc (start 183 104) (mid 181.828427 106.828427) (end 179 108) (stroke (width 0.2) (type solid)) (layer "Edge.Cuts"))
 (segment (start 168.23 96.52) (end 168.23 96.77) (width 0.25) (layer "F.Cu") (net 1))
 (segment (start 166 104) (end 166 100) (width 0.25) (layer "F.Cu") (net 1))
 (segment (start 166 100) (end 165.5 99.5) (width 0.25) (layer "F.Cu") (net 1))
 (segment (start 166 104) (end 165.800305 103.800305) (width 0.25) (layer "F.Cu") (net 1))
 (via (at 165.5 99.5) (size 0.8) (drill 0.4) (layers "F.Cu" "B.Cu") (free yes) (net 1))
 (segment (start 167.6 104) (end 171.1 104) (width 0.25) (layer "F.Cu") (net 2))
 (segment (start 171.48 96.52) (end 170.77 96.52) (width 0.25) (layer "F.Cu") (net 3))
 (segment (start 174 94) (end 171.48 96.52) (width 0.25) (layer "F.Cu") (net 3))
 (segment (start 176.5 85.39) (end 174 87.89) (width 0.25) (layer "F.Cu") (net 3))
 (segment (start 174 87.89) (end 174 94) (width 0.25) (layer "F.Cu") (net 3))
 (segment (start 176.5 96) (end 176.5 94) (width 0.25) (layer "F.Cu") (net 4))
 (segment (start 172.925 99.575) (end 176.5 96) (width 0.25) (layer "F.Cu") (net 4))
 (segment (start 172.925 104) (end 172.925 99.575) (width 0.25) (layer "F.Cu") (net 4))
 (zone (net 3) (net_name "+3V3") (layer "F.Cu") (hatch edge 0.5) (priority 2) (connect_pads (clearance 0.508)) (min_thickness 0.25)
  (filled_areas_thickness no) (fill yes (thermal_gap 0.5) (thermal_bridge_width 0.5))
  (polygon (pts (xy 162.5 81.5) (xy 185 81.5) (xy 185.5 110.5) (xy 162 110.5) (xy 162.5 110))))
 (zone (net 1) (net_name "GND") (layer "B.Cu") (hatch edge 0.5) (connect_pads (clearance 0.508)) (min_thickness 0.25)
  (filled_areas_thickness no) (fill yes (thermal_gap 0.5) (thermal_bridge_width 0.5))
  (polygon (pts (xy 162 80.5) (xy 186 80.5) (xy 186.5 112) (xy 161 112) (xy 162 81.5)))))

